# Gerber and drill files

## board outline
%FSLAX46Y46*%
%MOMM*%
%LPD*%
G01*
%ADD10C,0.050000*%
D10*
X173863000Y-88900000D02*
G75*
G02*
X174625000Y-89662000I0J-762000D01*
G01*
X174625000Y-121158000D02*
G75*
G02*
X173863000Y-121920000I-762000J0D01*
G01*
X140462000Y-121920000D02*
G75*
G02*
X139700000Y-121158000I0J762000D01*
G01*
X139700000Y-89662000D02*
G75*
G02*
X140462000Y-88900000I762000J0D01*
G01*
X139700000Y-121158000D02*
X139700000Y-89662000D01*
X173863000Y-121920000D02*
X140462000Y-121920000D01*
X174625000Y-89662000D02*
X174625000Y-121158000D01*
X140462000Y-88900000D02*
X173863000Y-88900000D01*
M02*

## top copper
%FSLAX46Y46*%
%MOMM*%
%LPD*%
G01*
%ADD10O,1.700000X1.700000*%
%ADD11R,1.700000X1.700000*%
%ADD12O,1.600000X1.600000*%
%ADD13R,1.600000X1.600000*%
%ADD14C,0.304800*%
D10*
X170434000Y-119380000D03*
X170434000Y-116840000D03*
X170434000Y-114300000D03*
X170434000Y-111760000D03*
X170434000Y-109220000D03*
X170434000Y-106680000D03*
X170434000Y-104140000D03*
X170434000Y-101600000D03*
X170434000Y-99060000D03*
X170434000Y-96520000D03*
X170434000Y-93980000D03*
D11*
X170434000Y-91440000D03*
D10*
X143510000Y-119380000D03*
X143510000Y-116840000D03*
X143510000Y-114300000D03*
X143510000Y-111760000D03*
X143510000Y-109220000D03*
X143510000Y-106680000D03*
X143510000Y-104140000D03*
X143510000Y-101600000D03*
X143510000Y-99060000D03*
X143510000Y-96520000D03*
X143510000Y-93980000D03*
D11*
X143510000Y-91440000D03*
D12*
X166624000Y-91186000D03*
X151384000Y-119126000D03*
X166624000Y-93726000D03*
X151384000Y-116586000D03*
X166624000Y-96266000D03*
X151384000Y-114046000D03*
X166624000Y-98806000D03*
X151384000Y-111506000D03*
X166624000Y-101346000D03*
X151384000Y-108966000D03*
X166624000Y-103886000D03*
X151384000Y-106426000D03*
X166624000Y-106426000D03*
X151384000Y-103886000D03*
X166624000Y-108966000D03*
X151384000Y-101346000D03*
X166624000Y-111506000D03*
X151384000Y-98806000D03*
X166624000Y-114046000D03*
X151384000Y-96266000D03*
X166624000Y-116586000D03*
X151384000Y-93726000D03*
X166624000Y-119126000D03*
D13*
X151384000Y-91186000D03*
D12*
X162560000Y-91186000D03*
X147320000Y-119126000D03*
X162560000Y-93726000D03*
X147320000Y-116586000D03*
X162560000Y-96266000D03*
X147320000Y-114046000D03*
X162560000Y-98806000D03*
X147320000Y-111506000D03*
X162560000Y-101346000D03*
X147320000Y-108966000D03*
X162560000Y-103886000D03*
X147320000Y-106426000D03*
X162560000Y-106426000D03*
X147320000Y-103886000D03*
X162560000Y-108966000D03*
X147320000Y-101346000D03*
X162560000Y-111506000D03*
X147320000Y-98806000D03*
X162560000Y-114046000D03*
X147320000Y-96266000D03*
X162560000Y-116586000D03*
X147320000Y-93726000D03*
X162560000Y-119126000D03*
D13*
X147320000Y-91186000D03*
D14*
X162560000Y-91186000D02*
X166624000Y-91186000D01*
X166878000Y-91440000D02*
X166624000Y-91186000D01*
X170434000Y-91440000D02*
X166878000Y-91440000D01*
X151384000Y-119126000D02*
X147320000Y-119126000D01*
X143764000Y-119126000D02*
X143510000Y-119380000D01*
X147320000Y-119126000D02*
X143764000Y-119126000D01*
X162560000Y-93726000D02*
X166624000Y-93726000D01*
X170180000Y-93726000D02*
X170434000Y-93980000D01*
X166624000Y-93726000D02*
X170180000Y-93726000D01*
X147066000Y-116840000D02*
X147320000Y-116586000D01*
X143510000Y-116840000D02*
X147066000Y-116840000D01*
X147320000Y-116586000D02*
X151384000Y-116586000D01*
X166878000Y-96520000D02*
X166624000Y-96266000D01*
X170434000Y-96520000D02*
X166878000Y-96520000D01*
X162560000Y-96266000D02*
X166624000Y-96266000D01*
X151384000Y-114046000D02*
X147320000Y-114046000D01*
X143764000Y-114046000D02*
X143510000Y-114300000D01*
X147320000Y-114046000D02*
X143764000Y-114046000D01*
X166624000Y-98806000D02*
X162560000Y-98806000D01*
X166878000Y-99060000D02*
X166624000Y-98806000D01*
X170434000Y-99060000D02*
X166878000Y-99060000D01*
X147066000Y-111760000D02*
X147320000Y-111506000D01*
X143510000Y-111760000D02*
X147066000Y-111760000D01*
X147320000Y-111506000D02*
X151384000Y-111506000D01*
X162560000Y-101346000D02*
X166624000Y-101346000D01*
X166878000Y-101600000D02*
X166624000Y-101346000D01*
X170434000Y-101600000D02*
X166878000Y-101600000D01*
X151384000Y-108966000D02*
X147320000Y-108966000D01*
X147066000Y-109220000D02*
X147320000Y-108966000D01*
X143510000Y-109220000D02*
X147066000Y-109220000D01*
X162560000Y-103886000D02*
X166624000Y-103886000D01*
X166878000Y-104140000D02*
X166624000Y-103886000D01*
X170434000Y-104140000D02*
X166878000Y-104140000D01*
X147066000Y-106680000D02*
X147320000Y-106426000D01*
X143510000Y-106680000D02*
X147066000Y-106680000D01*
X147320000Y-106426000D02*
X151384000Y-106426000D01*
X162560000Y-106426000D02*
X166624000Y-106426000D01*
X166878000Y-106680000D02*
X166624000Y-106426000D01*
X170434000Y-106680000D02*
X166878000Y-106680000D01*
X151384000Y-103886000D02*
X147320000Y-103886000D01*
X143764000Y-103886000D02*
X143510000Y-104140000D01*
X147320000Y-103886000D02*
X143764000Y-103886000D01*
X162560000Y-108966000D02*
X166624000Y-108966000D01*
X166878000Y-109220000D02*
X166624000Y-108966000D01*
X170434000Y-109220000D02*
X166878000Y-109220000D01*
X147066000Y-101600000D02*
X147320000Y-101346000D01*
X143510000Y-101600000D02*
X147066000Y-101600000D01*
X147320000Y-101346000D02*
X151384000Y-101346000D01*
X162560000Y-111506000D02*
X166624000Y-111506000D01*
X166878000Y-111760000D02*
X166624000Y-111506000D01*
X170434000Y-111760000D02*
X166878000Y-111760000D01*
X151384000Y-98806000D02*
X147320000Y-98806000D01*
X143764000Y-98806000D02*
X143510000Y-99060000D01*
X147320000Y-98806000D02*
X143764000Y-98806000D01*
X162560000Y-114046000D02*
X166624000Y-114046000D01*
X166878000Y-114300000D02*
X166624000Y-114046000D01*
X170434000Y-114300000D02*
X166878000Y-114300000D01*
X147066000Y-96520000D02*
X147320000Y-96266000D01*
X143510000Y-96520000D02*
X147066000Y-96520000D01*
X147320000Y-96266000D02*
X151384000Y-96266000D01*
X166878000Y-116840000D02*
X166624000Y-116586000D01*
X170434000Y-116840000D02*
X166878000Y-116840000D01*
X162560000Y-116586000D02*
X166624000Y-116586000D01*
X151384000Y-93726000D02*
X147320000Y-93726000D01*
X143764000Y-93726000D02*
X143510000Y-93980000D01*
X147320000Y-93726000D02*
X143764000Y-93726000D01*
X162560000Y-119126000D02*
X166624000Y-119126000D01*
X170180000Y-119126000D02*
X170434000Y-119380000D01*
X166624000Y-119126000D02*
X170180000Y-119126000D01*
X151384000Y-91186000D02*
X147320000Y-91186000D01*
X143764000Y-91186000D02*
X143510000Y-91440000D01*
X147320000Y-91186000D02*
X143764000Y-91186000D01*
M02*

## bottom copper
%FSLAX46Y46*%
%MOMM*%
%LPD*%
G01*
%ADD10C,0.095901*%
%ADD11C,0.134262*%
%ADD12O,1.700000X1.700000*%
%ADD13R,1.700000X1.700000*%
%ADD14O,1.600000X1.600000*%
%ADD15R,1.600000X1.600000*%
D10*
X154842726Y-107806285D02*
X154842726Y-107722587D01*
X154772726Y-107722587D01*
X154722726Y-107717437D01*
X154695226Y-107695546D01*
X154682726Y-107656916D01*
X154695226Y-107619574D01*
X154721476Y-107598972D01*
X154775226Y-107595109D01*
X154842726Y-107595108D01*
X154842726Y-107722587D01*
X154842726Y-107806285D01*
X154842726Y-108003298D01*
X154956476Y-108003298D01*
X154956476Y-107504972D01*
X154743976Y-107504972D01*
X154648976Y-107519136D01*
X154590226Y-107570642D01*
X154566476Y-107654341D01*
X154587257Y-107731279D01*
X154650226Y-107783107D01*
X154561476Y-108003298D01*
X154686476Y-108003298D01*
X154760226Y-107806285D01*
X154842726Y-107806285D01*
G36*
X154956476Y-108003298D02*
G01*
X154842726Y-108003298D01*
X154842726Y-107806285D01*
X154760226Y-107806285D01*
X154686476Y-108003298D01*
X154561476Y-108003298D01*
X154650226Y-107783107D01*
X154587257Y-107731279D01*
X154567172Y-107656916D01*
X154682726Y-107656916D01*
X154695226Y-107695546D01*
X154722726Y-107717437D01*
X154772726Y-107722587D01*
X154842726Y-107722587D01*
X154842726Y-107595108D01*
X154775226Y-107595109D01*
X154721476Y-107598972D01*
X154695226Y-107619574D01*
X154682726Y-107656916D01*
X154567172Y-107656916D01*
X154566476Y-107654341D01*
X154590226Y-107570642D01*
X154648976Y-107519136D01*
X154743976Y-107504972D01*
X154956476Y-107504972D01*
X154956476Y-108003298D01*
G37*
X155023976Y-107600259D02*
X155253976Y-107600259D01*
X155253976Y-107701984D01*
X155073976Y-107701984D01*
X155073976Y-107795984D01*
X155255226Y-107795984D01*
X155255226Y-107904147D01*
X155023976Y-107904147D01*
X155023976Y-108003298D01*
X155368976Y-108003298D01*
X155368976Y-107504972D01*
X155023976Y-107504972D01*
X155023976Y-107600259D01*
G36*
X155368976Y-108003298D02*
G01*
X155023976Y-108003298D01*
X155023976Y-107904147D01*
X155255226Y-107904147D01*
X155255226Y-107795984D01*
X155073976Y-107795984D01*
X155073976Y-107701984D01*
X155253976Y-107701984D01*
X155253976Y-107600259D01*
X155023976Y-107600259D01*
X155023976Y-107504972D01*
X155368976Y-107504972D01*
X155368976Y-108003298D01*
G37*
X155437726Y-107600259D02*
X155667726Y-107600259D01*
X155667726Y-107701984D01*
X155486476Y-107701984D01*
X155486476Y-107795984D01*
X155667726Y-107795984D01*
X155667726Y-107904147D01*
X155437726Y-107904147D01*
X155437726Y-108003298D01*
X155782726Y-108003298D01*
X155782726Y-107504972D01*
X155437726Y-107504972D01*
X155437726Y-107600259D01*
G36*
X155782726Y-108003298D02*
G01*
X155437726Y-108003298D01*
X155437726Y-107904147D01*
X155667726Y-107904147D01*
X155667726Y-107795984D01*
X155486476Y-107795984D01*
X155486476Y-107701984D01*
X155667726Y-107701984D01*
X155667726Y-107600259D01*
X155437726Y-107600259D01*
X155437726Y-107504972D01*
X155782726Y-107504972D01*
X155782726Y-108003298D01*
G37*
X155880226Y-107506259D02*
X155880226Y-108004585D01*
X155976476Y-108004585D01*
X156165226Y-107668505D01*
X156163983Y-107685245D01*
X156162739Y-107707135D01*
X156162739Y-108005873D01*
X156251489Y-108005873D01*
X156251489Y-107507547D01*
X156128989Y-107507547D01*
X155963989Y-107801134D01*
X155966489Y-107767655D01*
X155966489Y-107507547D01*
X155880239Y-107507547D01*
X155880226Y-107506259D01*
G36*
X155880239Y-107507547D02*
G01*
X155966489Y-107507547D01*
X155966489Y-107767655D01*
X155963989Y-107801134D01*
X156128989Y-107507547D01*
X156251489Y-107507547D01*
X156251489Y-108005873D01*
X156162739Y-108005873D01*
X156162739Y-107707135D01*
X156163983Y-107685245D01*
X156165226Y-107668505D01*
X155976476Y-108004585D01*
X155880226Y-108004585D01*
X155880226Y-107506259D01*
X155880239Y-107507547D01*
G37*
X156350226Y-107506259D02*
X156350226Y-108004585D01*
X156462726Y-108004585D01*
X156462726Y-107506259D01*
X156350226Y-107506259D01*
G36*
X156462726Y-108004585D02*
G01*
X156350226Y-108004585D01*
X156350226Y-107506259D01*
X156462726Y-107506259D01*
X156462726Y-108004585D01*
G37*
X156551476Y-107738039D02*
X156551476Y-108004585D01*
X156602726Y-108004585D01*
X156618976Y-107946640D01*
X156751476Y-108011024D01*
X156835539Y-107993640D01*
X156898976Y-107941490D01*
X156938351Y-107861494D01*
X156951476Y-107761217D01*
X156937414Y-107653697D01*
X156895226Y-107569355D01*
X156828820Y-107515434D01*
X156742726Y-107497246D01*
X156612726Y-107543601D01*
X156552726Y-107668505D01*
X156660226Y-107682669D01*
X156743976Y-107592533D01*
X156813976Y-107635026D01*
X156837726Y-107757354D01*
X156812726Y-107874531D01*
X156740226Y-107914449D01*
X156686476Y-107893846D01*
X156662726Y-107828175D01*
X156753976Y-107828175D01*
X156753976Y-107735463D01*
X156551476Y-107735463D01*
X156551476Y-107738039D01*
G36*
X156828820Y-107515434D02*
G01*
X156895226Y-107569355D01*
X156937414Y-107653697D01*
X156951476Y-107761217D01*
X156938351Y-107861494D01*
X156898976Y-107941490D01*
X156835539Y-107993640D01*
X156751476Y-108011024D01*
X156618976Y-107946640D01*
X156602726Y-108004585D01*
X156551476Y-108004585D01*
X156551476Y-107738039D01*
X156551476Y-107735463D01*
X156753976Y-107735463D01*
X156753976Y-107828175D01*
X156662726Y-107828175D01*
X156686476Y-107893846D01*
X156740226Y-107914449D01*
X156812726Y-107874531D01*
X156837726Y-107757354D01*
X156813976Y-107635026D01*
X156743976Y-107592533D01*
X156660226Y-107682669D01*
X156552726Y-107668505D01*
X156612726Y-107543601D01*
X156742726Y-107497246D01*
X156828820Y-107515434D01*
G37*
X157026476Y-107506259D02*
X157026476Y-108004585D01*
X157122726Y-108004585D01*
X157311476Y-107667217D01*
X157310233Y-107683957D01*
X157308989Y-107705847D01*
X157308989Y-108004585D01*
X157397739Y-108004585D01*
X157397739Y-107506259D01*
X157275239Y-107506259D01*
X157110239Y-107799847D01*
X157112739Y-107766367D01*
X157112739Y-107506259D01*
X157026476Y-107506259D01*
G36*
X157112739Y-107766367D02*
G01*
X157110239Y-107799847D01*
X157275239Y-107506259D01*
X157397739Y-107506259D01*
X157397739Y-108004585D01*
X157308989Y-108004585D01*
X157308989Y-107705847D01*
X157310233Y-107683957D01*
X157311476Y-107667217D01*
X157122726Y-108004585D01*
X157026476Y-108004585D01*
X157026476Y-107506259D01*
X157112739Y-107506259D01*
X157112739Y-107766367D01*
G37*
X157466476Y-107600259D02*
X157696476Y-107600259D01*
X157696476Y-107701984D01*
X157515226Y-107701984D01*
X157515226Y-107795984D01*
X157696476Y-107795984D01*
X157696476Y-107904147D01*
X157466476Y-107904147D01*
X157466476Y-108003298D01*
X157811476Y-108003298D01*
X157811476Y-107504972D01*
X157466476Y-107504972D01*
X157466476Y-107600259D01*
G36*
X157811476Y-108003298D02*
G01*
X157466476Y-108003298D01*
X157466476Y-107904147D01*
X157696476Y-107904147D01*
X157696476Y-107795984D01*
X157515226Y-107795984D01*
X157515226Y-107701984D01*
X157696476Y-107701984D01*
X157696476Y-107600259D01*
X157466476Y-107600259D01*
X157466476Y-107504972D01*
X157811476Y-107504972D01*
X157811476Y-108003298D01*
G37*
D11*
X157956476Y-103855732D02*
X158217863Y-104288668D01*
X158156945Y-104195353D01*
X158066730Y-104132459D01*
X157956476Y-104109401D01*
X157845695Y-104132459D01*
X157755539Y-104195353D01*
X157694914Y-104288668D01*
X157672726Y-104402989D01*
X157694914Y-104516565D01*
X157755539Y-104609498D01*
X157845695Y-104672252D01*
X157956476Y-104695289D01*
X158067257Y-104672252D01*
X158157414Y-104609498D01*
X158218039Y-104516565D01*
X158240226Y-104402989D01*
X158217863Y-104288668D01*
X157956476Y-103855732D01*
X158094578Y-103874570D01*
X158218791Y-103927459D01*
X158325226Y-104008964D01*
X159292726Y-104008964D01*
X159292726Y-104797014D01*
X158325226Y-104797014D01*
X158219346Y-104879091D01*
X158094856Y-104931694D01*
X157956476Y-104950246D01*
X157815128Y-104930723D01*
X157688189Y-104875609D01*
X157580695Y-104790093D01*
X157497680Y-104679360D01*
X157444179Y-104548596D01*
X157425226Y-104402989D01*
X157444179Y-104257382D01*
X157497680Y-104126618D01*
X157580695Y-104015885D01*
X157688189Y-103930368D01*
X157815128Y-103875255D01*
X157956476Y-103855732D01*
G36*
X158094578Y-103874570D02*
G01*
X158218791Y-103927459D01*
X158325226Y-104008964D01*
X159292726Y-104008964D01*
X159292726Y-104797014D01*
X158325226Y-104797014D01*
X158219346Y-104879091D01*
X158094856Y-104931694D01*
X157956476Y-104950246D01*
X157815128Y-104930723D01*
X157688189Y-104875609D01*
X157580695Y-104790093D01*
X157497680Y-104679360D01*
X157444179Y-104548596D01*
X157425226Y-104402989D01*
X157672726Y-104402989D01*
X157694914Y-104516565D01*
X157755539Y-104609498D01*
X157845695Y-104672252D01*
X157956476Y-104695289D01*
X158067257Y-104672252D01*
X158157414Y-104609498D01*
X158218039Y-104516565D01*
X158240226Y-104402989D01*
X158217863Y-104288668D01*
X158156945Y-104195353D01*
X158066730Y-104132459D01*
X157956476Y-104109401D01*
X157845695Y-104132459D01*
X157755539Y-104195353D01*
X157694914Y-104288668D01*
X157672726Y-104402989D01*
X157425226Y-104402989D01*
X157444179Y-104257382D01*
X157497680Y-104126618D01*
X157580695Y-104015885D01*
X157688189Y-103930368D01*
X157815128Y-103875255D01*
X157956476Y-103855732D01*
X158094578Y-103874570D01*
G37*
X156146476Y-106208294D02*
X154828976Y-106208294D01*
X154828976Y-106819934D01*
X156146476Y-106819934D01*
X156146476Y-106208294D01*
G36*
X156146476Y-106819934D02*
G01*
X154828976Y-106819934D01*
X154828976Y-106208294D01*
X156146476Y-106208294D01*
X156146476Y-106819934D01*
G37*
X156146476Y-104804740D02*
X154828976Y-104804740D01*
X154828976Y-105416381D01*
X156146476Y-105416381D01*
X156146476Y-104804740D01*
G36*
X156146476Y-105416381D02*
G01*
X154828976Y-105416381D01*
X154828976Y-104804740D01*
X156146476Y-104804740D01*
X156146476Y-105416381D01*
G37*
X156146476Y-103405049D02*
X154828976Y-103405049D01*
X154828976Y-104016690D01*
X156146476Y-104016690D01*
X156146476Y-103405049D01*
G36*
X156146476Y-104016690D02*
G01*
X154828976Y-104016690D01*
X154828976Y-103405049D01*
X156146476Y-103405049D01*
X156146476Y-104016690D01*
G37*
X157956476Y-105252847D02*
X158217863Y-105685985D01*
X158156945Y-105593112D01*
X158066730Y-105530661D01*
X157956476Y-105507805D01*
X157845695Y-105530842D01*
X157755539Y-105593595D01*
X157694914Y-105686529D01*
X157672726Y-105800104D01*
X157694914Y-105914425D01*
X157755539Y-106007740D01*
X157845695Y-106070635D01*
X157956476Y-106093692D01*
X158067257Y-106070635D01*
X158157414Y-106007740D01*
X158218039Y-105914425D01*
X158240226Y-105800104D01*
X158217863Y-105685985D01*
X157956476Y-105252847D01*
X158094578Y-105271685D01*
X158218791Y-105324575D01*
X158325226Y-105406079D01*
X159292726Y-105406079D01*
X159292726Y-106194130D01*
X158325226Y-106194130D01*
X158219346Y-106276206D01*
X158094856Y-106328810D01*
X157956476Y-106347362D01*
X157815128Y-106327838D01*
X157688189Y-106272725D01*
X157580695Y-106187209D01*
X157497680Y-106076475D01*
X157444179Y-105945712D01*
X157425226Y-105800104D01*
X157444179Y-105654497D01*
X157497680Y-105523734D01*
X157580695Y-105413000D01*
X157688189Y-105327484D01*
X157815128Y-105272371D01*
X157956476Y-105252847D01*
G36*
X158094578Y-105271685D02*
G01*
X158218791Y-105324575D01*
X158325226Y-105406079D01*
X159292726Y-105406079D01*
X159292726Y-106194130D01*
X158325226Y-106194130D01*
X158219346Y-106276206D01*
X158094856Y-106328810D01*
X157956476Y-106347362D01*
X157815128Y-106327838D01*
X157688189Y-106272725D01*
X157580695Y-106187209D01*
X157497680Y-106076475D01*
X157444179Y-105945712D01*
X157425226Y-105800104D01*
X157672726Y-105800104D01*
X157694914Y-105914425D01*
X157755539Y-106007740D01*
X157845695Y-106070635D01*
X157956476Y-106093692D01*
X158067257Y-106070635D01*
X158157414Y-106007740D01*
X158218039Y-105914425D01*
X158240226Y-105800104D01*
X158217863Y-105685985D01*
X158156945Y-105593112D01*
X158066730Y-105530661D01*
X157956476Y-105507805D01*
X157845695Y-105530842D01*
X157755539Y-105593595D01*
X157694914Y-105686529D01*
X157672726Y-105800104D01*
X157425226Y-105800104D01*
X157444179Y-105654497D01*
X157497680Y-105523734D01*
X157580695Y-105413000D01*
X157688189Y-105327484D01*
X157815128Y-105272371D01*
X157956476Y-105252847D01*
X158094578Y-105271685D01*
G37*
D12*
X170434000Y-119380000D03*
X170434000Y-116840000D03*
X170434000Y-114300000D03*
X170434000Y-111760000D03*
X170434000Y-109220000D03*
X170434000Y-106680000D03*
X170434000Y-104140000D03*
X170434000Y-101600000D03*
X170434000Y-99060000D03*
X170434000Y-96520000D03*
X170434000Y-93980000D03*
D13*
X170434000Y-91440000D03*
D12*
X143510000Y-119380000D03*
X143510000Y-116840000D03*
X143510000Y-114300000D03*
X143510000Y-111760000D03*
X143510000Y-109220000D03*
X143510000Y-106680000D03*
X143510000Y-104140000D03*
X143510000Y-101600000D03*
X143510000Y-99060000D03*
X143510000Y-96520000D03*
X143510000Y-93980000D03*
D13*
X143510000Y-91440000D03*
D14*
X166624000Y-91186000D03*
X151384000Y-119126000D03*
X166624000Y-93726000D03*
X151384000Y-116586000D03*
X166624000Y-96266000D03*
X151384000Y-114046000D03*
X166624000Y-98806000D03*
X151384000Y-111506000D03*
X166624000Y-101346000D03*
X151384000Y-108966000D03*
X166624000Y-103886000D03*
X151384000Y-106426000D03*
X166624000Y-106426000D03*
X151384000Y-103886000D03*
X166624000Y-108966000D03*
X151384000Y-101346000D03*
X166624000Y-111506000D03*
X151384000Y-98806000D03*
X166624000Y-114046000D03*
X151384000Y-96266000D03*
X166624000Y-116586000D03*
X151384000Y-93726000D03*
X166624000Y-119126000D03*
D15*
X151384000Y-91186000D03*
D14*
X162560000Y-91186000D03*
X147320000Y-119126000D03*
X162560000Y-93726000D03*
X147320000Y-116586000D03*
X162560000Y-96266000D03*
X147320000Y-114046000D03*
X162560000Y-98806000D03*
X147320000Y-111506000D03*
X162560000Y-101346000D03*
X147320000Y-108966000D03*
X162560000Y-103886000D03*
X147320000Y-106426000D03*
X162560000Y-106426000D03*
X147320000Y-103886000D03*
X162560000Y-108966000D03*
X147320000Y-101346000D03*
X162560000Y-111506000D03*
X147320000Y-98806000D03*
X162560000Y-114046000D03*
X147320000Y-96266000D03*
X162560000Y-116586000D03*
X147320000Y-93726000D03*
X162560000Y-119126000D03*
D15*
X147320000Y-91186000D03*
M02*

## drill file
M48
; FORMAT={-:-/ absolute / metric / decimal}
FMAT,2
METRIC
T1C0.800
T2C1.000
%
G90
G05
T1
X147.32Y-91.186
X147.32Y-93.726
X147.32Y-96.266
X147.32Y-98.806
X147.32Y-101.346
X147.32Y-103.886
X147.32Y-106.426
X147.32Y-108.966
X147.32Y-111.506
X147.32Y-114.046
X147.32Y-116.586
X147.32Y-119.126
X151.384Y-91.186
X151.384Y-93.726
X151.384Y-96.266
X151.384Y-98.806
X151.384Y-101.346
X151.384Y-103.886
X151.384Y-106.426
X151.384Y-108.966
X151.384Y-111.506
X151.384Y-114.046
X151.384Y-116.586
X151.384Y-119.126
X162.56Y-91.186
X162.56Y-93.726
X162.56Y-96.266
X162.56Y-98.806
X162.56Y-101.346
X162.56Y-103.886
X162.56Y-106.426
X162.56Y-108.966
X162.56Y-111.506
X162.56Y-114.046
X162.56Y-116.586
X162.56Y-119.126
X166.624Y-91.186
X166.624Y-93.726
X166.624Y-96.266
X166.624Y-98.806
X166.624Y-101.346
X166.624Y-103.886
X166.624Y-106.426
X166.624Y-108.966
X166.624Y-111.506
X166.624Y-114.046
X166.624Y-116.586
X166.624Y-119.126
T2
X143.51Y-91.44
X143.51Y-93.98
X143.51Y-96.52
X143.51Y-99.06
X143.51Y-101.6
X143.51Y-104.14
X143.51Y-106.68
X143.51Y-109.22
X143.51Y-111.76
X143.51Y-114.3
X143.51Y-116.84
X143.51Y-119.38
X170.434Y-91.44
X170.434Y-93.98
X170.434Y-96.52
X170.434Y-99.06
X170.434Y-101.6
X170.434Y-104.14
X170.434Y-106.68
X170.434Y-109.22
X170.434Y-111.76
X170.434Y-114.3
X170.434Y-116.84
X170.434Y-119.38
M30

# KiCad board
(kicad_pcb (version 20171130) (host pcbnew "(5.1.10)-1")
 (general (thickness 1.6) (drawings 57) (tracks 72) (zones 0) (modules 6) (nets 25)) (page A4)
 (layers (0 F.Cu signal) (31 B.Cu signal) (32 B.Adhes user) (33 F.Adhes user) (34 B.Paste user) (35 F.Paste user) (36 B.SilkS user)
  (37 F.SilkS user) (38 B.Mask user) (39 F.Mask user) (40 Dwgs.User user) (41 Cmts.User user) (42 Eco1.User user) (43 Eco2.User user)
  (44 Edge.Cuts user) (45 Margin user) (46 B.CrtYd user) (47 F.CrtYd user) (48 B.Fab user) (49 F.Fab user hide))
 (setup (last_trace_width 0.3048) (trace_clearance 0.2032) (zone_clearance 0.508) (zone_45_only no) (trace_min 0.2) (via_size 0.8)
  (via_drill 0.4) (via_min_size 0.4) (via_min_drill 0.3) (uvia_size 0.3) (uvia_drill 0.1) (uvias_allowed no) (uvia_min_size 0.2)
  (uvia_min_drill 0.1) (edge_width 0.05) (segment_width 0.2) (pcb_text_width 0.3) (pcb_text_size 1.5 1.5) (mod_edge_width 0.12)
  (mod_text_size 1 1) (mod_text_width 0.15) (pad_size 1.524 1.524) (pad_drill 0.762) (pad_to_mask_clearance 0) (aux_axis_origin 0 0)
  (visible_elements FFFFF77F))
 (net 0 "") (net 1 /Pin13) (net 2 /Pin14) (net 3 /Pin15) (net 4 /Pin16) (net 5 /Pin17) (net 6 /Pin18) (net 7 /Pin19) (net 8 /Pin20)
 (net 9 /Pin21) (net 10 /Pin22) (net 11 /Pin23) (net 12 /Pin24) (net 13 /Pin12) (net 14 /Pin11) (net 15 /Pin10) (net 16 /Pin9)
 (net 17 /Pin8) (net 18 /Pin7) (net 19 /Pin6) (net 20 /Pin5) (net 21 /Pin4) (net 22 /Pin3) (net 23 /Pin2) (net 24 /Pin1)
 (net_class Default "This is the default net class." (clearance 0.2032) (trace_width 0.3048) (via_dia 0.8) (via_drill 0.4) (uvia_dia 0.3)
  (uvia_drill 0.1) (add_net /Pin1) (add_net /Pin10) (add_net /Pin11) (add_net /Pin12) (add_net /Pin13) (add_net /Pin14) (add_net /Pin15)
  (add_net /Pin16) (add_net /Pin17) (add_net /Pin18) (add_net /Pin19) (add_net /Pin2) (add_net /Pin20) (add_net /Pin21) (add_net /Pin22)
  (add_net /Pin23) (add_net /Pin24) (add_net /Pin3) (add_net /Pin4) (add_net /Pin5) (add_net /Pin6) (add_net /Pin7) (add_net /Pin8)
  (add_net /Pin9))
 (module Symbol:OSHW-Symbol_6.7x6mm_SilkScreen (layer B.Cu) (at 157.0736 95.6818 180)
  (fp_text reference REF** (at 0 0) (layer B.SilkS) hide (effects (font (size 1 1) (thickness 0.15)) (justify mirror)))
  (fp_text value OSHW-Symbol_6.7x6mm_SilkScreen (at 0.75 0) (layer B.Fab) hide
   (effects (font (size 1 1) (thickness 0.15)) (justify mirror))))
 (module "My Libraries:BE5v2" (layer B.Cu) (at 159.561476 103.011024 180)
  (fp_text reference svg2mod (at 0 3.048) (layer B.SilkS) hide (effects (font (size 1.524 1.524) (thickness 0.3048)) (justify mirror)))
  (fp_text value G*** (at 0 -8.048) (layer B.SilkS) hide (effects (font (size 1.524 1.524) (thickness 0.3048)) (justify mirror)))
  (fp_poly
   (pts (xy 4.71875 -4.795261) (xy 4.71875 -4.711563) (xy 4.78875 -4.711563) (xy 4.83875 -4.706413) (xy 4.86625 -4.684522)
    (xy 4.87875 -4.645892) (xy 4.86625 -4.60855) (xy 4.84 -4.587948) (xy 4.78625 -4.584085) (xy 4.71875 -4.584084) (xy 4.71875 -4.711563)
    (xy 4.71875 -4.795261) (xy 4.71875 -4.992274) (xy 4.605 -4.992274) (xy 4.605 -4.493948) (xy 4.8175 -4.493948) (xy 4.9125 -4.508112)
    (xy 4.97125 -4.559618) (xy 4.995 -4.643317) (xy 4.974219 -4.720255) (xy 4.91125 -4.772083) (xy 5 -4.992274) (xy 4.875 -4.992274)
    (xy 4.80125 -4.795261) (xy 4.71875 -4.795261))
   (layer B.Cu) (width 0.095901))
  (fp_poly
   (pts (xy 4.5375 -4.589235) (xy 4.3075 -4.589235) (xy 4.3075 -4.69096) (xy 4.4875 -4.69096) (xy 4.4875 -4.78496) (xy 4.30625 -4.78496)
    (xy 4.30625 -4.893123) (xy 4.5375 -4.893123) (xy 4.5375 -4.992274) (xy 4.1925 -4.992274) (xy 4.1925 -4.493948) (xy 4.5375 -4.493948)
    (xy 4.5375 -4.589235))
   (layer B.Cu) (width 0.095901))
  (fp_poly
   (pts (xy 4.12375 -4.589235) (xy 3.89375 -4.589235) (xy 3.89375 -4.69096) (xy 4.075 -4.69096) (xy 4.075 -4.78496) (xy 3.89375 -4.78496)
    (xy 3.89375 -4.893123) (xy 4.12375 -4.893123) (xy 4.12375 -4.992274) (xy 3.77875 -4.992274) (xy 3.77875 -4.493948)
    (xy 4.12375 -4.493948) (xy 4.12375 -4.589235))
   (layer B.Cu) (width 0.095901))
  (fp_poly
   (pts (xy 3.68125 -4.495235) (xy 3.68125 -4.993561) (xy 3.585 -4.993561) (xy 3.39625 -4.657481) (xy 3.397493 -4.674221)
    (xy 3.398737 -4.696111) (xy 3.398737 -4.994849) (xy 3.309987 -4.994849) (xy 3.309987 -4.496523) (xy 3.432487 -4.496523)
    (xy 3.597487 -4.79011) (xy 3.594987 -4.756631) (xy 3.594987 -4.496523) (xy 3.681237 -4.496523) (xy 3.68125 -4.495235))
   (layer B.Cu) (width 0.095901))
  (fp_poly
   (pts (xy 3.21125 -4.495235) (xy 3.21125 -4.993561) (xy 3.09875 -4.993561) (xy 3.09875 -4.495235) (xy 3.21125 -4.495235)) (layer B.Cu)
   (width 0.095901))
  (fp_poly
   (pts (xy 3.01 -4.727015) (xy 3.01 -4.993561) (xy 2.95875 -4.993561) (xy 2.9425 -4.935616) (xy 2.81 -5) (xy 2.725937 -4.982616)
    (xy 2.6625 -4.930466) (xy 2.623125 -4.85047) (xy 2.61 -4.750193) (xy 2.624062 -4.642673) (xy 2.66625 -4.558331) (xy 2.732656 -4.50441)
    (xy 2.81875 -4.486222) (xy 2.94875 -4.532577) (xy 3.00875 -4.657481) (xy 2.90125 -4.671645) (xy 2.8175 -4.581509) (xy 2.7475 -4.624002)
    (xy 2.72375 -4.74633) (xy 2.74875 -4.863507) (xy 2.82125 -4.903425) (xy 2.875 -4.882822) (xy 2.89875 -4.817151) (xy 2.8075 -4.817151)
    (xy 2.8075 -4.724439) (xy 3.01 -4.724439) (xy 3.01 -4.727015))
   (layer B.Cu) (width 0.095901))
  (fp_poly
   (pts (xy 2.535 -4.495235) (xy 2.535 -4.993561) (xy 2.43875 -4.993561) (xy 2.25 -4.656193) (xy 2.251243 -4.672933) (xy 2.252487 -4.694823)
    (xy 2.252487 -4.993561) (xy 2.163737 -4.993561) (xy 2.163737 -4.495235) (xy 2.286237 -4.495235) (xy 2.451237 -4.788823)
    (xy 2.448737 -4.755343) (xy 2.448737 -4.495235) (xy 2.535 -4.495235))
   (layer B.Cu) (width 0.095901))
  (fp_poly
   (pts (xy 2.095 -4.589235) (xy 1.865 -4.589235) (xy 1.865 -4.69096) (xy 2.04625 -4.69096) (xy 2.04625 -4.78496) (xy 1.865 -4.78496)
    (xy 1.865 -4.893123) (xy 2.095 -4.893123) (xy 2.095 -4.992274) (xy 1.75 -4.992274) (xy 1.75 -4.493948) (xy 2.095 -4.493948)
    (xy 2.095 -4.589235))
   (layer B.Cu) (width 0.095901))
  (fp_poly
   (pts (xy 1.605 -0.844708) (xy 1.343613 -1.277644) (xy 1.404531 -1.184329) (xy 1.494746 -1.121435) (xy 1.605 -1.098377)
    (xy 1.715781 -1.121435) (xy 1.805937 -1.184329) (xy 1.866562 -1.277644) (xy 1.88875 -1.391965) (xy 1.866562 -1.505541)
    (xy 1.805937 -1.598474) (xy 1.715781 -1.661228) (xy 1.605 -1.684265) (xy 1.494219 -1.661228) (xy 1.404062 -1.598474)
    (xy 1.343437 -1.505541) (xy 1.32125 -1.391965) (xy 1.343613 -1.277644) (xy 1.605 -0.844708) (xy 1.466898 -0.863546)
    (xy 1.342685 -0.916435) (xy 1.23625 -0.99794) (xy 0.26875 -0.99794) (xy 0.26875 -1.78599) (xy 1.23625 -1.78599) (xy 1.34213 -1.868067)
    (xy 1.46662 -1.92067) (xy 1.605 -1.939222) (xy 1.746348 -1.919699) (xy 1.873287 -1.864585) (xy 1.980781 -1.779069)
    (xy 2.063796 -1.668336) (xy 2.117297 -1.537572) (xy 2.13625 -1.391965) (xy 2.117297 -1.246358) (xy 2.063796 -1.115594)
    (xy 1.980781 -1.004861) (xy 1.873287 -0.919344) (xy 1.746348 -0.864231) (xy 1.605 -0.844708))
   (layer B.Cu) (width 0.134262))
  (fp_poly
   (pts (xy 3.415 -3.19727) (xy 4.7325 -3.19727) (xy 4.7325 -3.80891) (xy 3.415 -3.80891) (xy 3.415 -3.19727)) (layer B.Cu) (width 0.134262))
  (fp_poly
   (pts (xy 3.415 -1.793716) (xy 4.7325 -1.793716) (xy 4.7325 -2.405357) (xy 3.415 -2.405357) (xy 3.415 -1.793716)) (layer B.Cu)
   (width 0.134262))
  (fp_poly
   (pts (xy 3.415 -0.394025) (xy 4.7325 -0.394025) (xy 4.7325 -1.005666) (xy 3.415 -1.005666) (xy 3.415 -0.394025)) (layer B.Cu)
   (width 0.134262))
  (fp_poly
   (pts (xy 1.605 -2.241823) (xy 1.343613 -2.674961) (xy 1.404531 -2.582088) (xy 1.494746 -2.519637) (xy 1.605 -2.496781)
    (xy 1.715781 -2.519818) (xy 1.805937 -2.582571) (xy 1.866562 -2.675505) (xy 1.88875 -2.78908) (xy 1.866562 -2.903401)
    (xy 1.805937 -2.996716) (xy 1.715781 -3.059611) (xy 1.605 -3.082668) (xy 1.494219 -3.059611) (xy 1.404062 -2.996716)
    (xy 1.343437 -2.903401) (xy 1.32125 -2.78908) (xy 1.343613 -2.674961) (xy 1.605 -2.241823) (xy 1.466898 -2.260661)
    (xy 1.342685 -2.313551) (xy 1.23625 -2.395055) (xy 0.26875 -2.395055) (xy 0.26875 -3.183106) (xy 1.23625 -3.183106)
    (xy 1.34213 -3.265182) (xy 1.46662 -3.317786) (xy 1.605 -3.336338) (xy 1.746348 -3.316814) (xy 1.873287 -3.261701)
    (xy 1.980781 -3.176185) (xy 2.063796 -3.065451) (xy 2.117297 -2.934688) (xy 2.13625 -2.78908) (xy 2.117297 -2.643473)
    (xy 2.063796 -2.51271) (xy 1.980781 -2.401976) (xy 1.873287 -2.31646) (xy 1.746348 -2.261347) (xy 1.605 -2.241823))
   (layer B.Cu) (width 0.134262)))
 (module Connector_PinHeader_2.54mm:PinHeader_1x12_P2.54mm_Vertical (layer F.Cu) (at 170.434 91.44)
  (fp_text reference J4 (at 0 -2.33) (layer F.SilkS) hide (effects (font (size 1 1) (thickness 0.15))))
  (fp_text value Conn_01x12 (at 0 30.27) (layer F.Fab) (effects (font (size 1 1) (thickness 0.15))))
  (pad 12 thru_hole oval (at 0 27.94) (size 1.7 1.7) (drill 1) (layers *.Cu *.Mask) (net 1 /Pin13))
  (pad 11 thru_hole oval (at 0 25.4) (size 1.7 1.7) (drill 1) (layers *.Cu *.Mask) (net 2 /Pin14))
  (pad 10 thru_hole oval (at 0 22.86) (size 1.7 1.7) (drill 1) (layers *.Cu *.Mask) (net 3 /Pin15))
  (pad 9 thru_hole oval (at 0 20.32) (size 1.7 1.7) (drill 1) (layers *.Cu *.Mask) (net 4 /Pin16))
  (pad 8 thru_hole oval (at 0 17.78) (size 1.7 1.7) (drill 1) (layers *.Cu *.Mask) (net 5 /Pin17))
  (pad 7 thru_hole oval (at 0 15.24) (size 1.7 1.7) (drill 1) (layers *.Cu *.Mask) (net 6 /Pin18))
  (pad 6 thru_hole oval (at 0 12.7) (size 1.7 1.7) (drill 1) (layers *.Cu *.Mask) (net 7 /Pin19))
  (pad 5 thru_hole oval (at 0 10.16) (size 1.7 1.7) (drill 1) (layers *.Cu *.Mask) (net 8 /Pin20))
  (pad 4 thru_hole oval (at 0 7.62) (size 1.7 1.7) (drill 1) (layers *.Cu *.Mask) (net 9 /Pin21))
  (pad 3 thru_hole oval (at 0 5.08) (size 1.7 1.7) (drill 1) (layers *.Cu *.Mask) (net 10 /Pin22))
  (pad 2 thru_hole oval (at 0 2.54) (size 1.7 1.7) (drill 1) (layers *.Cu *.Mask) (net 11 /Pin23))
  (pad 1 thru_hole rect (at 0 0) (size 1.7 1.7) (drill 1) (layers *.Cu *.Mask) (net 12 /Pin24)))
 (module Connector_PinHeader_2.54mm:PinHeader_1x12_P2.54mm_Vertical (layer F.Cu) (at 143.51 91.44)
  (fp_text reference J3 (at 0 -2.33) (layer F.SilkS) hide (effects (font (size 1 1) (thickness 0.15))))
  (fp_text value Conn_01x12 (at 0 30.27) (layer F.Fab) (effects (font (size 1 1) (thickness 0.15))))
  (pad 12 thru_hole oval (at 0 27.94) (size 1.7 1.7) (drill 1) (layers *.Cu *.Mask) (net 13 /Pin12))
  (pad 11 thru_hole oval (at 0 25.4) (size 1.7 1.7) (drill 1) (layers *.Cu *.Mask) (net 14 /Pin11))
  (pad 10 thru_hole oval (at 0 22.86) (size 1.7 1.7) (drill 1) (layers *.Cu *.Mask) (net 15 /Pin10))
  (pad 9 thru_hole oval (at 0 20.32) (size 1.7 1.7) (drill 1) (layers *.Cu *.Mask) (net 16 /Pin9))
  (pad 8 thru_hole oval (at 0 17.78) (size 1.7 1.7) (drill 1) (layers *.Cu *.Mask) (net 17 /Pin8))
  (pad 7 thru_hole oval (at 0 15.24) (size 1.7 1.7) (drill 1) (layers *.Cu *.Mask) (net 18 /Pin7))
  (pad 6 thru_hole oval (at 0 12.7) (size 1.7 1.7) (drill 1) (layers *.Cu *.Mask) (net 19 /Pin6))
  (pad 5 thru_hole oval (at 0 10.16) (size 1.7 1.7) (drill 1) (layers *.Cu *.Mask) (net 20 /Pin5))
  (pad 4 thru_hole oval (at 0 7.62) (size 1.7 1.7) (drill 1) (layers *.Cu *.Mask) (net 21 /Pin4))
  (pad 3 thru_hole oval (at 0 5.08) (size 1.7 1.7) (drill 1) (layers *.Cu *.Mask) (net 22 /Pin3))
  (pad 2 thru_hole oval (at 0 2.54) (size 1.7 1.7) (drill 1) (layers *.Cu *.Mask) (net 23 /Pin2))
  (pad 1 thru_hole rect (at 0 0) (size 1.7 1.7) (drill 1) (layers *.Cu *.Mask) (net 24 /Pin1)))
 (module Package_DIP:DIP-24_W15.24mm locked (layer F.Cu) (at 151.384 91.186)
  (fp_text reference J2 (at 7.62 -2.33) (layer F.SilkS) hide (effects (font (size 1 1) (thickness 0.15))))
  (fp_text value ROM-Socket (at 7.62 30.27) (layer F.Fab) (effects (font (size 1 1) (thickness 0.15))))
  (pad 24 thru_hole oval (at 15.24 0) (size 1.6 1.6) (drill 0.8) (layers *.Cu *.Mask) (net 12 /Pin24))
  (pad 12 thru_hole oval (at 0 27.94) (size 1.6 1.6) (drill 0.8) (layers *.Cu *.Mask) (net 13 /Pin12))
  (pad 23 thru_hole oval (at 15.24 2.54) (size 1.6 1.6) (drill 0.8) (layers *.Cu *.Mask) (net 11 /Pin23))
  (pad 11 thru_hole oval (at 0 25.4) (size 1.6 1.6) (drill 0.8) (layers *.Cu *.Mask) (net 14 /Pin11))
  (pad 22 thru_hole oval (at 15.24 5.08) (size 1.6 1.6) (drill 0.8) (layers *.Cu *.Mask) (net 10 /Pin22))
  (pad 10 thru_hole oval (at 0 22.86) (size 1.6 1.6) (drill 0.8) (layers *.Cu *.Mask) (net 15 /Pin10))
  (pad 21 thru_hole oval (at 15.24 7.62) (size 1.6 1.6) (drill 0.8) (layers *.Cu *.Mask) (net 9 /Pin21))
  (pad 9 thru_hole oval (at 0 20.32) (size 1.6 1.6) (drill 0.8) (layers *.Cu *.Mask) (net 16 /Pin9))
  (pad 20 thru_hole oval (at 15.24 10.16) (size 1.6 1.6) (drill 0.8) (layers *.Cu *.Mask) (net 8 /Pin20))
  (pad 8 thru_hole oval (at 0 17.78) (size 1.6 1.6) (drill 0.8) (layers *.Cu *.Mask) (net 17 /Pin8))
  (pad 19 thru_hole oval (at 15.24 12.7) (size 1.6 1.6) (drill 0.8) (layers *.Cu *.Mask) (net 7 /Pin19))
  (pad 7 thru_hole oval (at 0 15.24) (size 1.6 1.6) (drill 0.8) (layers *.Cu *.Mask) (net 18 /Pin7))
  (pad 18 thru_hole oval (at 15.24 15.24) (size 1.6 1.6) (drill 0.8) (layers *.Cu *.Mask) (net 6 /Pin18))
  (pad 6 thru_hole oval (at 0 12.7) (size 1.6 1.6) (drill 0.8) (layers *.Cu *.Mask) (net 19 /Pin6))
  (pad 17 thru_hole oval (at 15.24 17.78) (size 1.6 1.6) (drill 0.8) (layers *.Cu *.Mask) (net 5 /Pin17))
  (pad 5 thru_hole oval (at 0 10.16) (size 1.6 1.6) (drill 0.8) (layers *.Cu *.Mask) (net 20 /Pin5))
  (pad 16 thru_hole oval (at 15.24 20.32) (size 1.6 1.6) (drill 0.8) (layers *.Cu *.Mask) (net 4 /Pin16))
  (pad 4 thru_hole oval (at 0 7.62) (size 1.6 1.6) (drill 0.8) (layers *.Cu *.Mask) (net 21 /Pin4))
  (pad 15 thru_hole oval (at 15.24 22.86) (size 1.6 1.6) (drill 0.8) (layers *.Cu *.Mask) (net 3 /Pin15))
  (pad 3 thru_hole oval (at 0 5.08) (size 1.6 1.6) (drill 0.8) (layers *.Cu *.Mask) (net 22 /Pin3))
  (pad 14 thru_hole oval (at 15.24 25.4) (size 1.6 1.6) (drill 0.8) (layers *.Cu *.Mask) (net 2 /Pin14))
  (pad 2 thru_hole oval (at 0 2.54) (size 1.6 1.6) (drill 0.8) (layers *.Cu *.Mask) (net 23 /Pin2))
  (pad 13 thru_hole oval (at 15.24 27.94) (size 1.6 1.6) (drill 0.8) (layers *.Cu *.Mask) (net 1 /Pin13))
  (pad 1 thru_hole rect (at 0 0) (size 1.6 1.6) (drill 0.8) (layers *.Cu *.Mask) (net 24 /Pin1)))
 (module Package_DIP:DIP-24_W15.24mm (layer F.Cu) (at 147.32 91.186)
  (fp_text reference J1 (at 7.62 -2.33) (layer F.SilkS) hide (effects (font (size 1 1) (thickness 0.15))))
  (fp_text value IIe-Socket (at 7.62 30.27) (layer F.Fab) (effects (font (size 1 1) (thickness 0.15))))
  (pad 24 thru_hole oval (at 15.24 0) (size 1.6 1.6) (drill 0.8) (layers *.Cu *.Mask) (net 12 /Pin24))
  (pad 12 thru_hole oval (at 0 27.94) (size 1.6 1.6) (drill 0.8) (layers *.Cu *.Mask) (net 13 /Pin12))
  (pad 23 thru_hole oval (at 15.24 2.54) (size 1.6 1.6) (drill 0.8) (layers *.Cu *.Mask) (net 11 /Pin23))
  (pad 11 thru_hole oval (at 0 25.4) (size 1.6 1.6) (drill 0.8) (layers *.Cu *.Mask) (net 14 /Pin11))
  (pad 22 thru_hole oval (at 15.24 5.08) (size 1.6 1.6) (drill 0.8) (layers *.Cu *.Mask) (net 10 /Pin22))
  (pad 10 thru_hole oval (at 0 22.86) (size 1.6 1.6) (drill 0.8) (layers *.Cu *.Mask) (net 15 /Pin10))
  (pad 21 thru_hole oval (at 15.24 7.62) (size 1.6 1.6) (drill 0.8) (layers *.Cu *.Mask) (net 9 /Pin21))
  (pad 9 thru_hole oval (at 0 20.32) (size 1.6 1.6) (drill 0.8) (layers *.Cu *.Mask) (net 16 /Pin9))
  (pad 20 thru_hole oval (at 15.24 10.16) (size 1.6 1.6) (drill 0.8) (layers *.Cu *.Mask) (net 8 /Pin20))
  (pad 8 thru_hole oval (at 0 17.78) (size 1.6 1.6) (drill 0.8) (layers *.Cu *.Mask) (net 17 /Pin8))
  (pad 19 thru_hole oval (at 15.24 12.7) (size 1.6 1.6) (drill 0.8) (layers *.Cu *.Mask) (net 7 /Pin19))
  (pad 7 thru_hole oval (at 0 15.24) (size 1.6 1.6) (drill 0.8) (layers *.Cu *.Mask) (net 18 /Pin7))
  (pad 18 thru_hole oval (at 15.24 15.24) (size 1.6 1.6) (drill 0.8) (layers *.Cu *.Mask) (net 6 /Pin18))
  (pad 6 thru_hole oval (at 0 12.7) (size 1.6 1.6) (drill 0.8) (layers *.Cu *.Mask) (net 19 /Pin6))
  (pad 17 thru_hole oval (at 15.24 17.78) (size 1.6 1.6) (drill 0.8) (layers *.Cu *.Mask) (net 5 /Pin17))
  (pad 5 thru_hole oval (at 0 10.16) (size 1.6 1.6) (drill 0.8) (layers *.Cu *.Mask) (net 20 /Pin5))
  (pad 16 thru_hole oval (at 15.24 20.32) (size 1.6 1.6) (drill 0.8) (layers *.Cu *.Mask) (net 4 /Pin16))
  (pad 4 thru_hole oval (at 0 7.62) (size 1.6 1.6) (drill 0.8) (layers *.Cu *.Mask) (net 21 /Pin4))
  (pad 15 thru_hole oval (at 15.24 22.86) (size 1.6 1.6) (drill 0.8) (layers *.Cu *.Mask) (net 3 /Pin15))
  (pad 3 thru_hole oval (at 0 5.08) (size 1.6 1.6) (drill 0.8) (layers *.Cu *.Mask) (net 22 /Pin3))
  (pad 14 thru_hole oval (at 15.24 25.4) (size 1.6 1.6) (drill 0.8) (layers *.Cu *.Mask) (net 2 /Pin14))
  (pad 2 thru_hole oval (at 0 2.54) (size 1.6 1.6) (drill 0.8) (layers *.Cu *.Mask) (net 23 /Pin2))
  (pad 13 thru_hole oval (at 15.24 27.94) (size 1.6 1.6) (drill 0.8) (layers *.Cu *.Mask) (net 1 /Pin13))
  (pad 1 thru_hole rect (at 0 0) (size 1.6 1.6) (drill 0.8) (layers *.Cu *.Mask) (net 24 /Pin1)))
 (gr_arc (start 173.863 89.662) (end 174.625 89.662) (angle -90) (layer Edge.Cuts) (width 0.05))
 (gr_arc (start 173.863 121.158) (end 173.863 121.92) (angle -90) (layer Edge.Cuts) (width 0.05))
 (gr_arc (start 140.462 121.158) (end 139.7 121.158) (angle -90) (layer Edge.Cuts) (width 0.05))
 (gr_arc (start 140.462 89.662) (end 140.462 88.9) (angle -90) (layer Edge.Cuts) (width 0.05))
 (gr_line (start 139.7 121.158) (end 139.7 89.662) (layer Edge.Cuts) (width 0.05))
 (gr_line (start 173.863 121.92) (end 140.462 121.92) (layer Edge.Cuts) (width 0.05))
 (gr_line (start 174.625 89.662) (end 174.625 121.158) (layer Edge.Cuts) (width 0.05))
 (gr_line (start 140.462 88.9) (end 173.863 88.9) (layer Edge.Cuts) (width 0.05))
 (segment (start 162.56 91.186) (end 166.624 91.186) (width 0.3048) (layer F.Cu) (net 12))
 (segment (start 166.878 91.44) (end 166.624 91.186) (width 0.3048) (layer F.Cu) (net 12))
 (segment (start 170.434 91.44) (end 166.878 91.44) (width 0.3048) (layer F.Cu) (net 12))
 (segment (start 151.384 119.126) (end 147.32 119.126) (width 0.3048) (layer F.Cu) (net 13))
 (segment (start 143.764 119.126) (end 143.51 119.38) (width 0.3048) (layer F.Cu) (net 13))
 (segment (start 147.32 119.126) (end 143.764 119.126) (width 0.3048) (layer F.Cu) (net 13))
 (segment (start 162.56 93.726) (end 166.624 93.726) (width 0.3048) (layer F.Cu) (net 11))
 (segment (start 170.18 93.726) (end 170.434 93.98) (width 0.3048) (layer F.Cu) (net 11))
 (segment (start 166.624 93.726) (end 170.18 93.726) (width 0.3048) (layer F.Cu) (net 11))
 (segment (start 147.066 116.84) (end 147.32 116.586) (width 0.3048) (layer F.Cu) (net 14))
 (segment (start 143.51 116.84) (end 147.066 116.84) (width 0.3048) (layer F.Cu) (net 14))
 (segment (start 147.32 116.586) (end 151.384 116.586) (width 0.3048) (layer F.Cu) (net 14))
 (segment (start 166.878 96.52) (end 166.624 96.266) (width 0.3048) (layer F.Cu) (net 10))
 (segment (start 170.434 96.52) (end 166.878 96.52) (width 0.3048) (layer F.Cu) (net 10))
 (segment (start 162.56 96.266) (end 166.624 96.266) (width 0.3048) (layer F.Cu) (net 10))
 (segment (start 151.384 114.046) (end 147.32 114.046) (width 0.3048) (layer F.Cu) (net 15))
 (segment (start 143.764 114.046) (end 143.51 114.3) (width 0.3048) (layer F.Cu) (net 15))
 (segment (start 147.32 114.046) (end 143.764 114.046) (width 0.3048) (layer F.Cu) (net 15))
 (segment (start 166.624 98.806) (end 162.56 98.806) (width 0.3048) (layer F.Cu) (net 9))
 (segment (start 166.878 99.06) (end 166.624 98.806) (width 0.3048) (layer F.Cu) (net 9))
 (segment (start 170.434 99.06) (end 166.878 99.06) (width 0.3048) (layer F.Cu) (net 9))
 (segment (start 147.066 111.76) (end 147.32 111.506) (width 0.3048) (layer F.Cu) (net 16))
 (segment (start 143.51 111.76) (end 147.066 111.76) (width 0.3048) (layer F.Cu) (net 16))
 (segment (start 147.32 111.506) (end 151.384 111.506) (width 0.3048) (layer F.Cu) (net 16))
 (segment (start 162.56 101.346) (end 166.624 101.346) (width 0.3048) (layer F.Cu) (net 8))
 (segment (start 166.878 101.6) (end 166.624 101.346) (width 0.3048) (layer F.Cu) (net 8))
 (segment (start 170.434 101.6) (end 166.878 101.6) (width 0.3048) (layer F.Cu) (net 8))
 (segment (start 151.384 108.966) (end 147.32 108.966) (width 0.3048) (layer F.Cu) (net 17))
 (segment (start 147.066 109.22) (end 147.32 108.966) (width 0.3048) (layer F.Cu) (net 17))
 (segment (start 143.51 109.22) (end 147.066 109.22) (width 0.3048) (layer F.Cu) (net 17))
 (segment (start 162.56 103.886) (end 166.624 103.886) (width 0.3048) (layer F.Cu) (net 7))
 (segment (start 166.878 104.14) (end 166.624 103.886) (width 0.3048) (layer F.Cu) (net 7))
 (segment (start 170.434 104.14) (end 166.878 104.14) (width 0.3048) (layer F.Cu) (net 7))
 (segment (start 147.066 106.68) (end 147.32 106.426) (width 0.3048) (layer F.Cu) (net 18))
 (segment (start 143.51 106.68) (end 147.066 106.68) (width 0.3048) (layer F.Cu) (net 18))
 (segment (start 147.32 106.426) (end 151.384 106.426) (width 0.3048) (layer F.Cu) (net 18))
 (segment (start 162.56 106.426) (end 166.624 106.426) (width 0.3048) (layer F.Cu) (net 6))
 (segment (start 166.878 106.68) (end 166.624 106.426) (width 0.3048) (layer F.Cu) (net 6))
 (segment (start 170.434 106.68) (end 166.878 106.68) (width 0.3048) (layer F.Cu) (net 6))
 (segment (start 151.384 103.886) (end 147.32 103.886) (width 0.3048) (layer F.Cu) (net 19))
 (segment (start 143.764 103.886) (end 143.51 104.14) (width 0.3048) (layer F.Cu) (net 19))
 (segment (start 147.32 103.886) (end 143.764 103.886) (width 0.3048) (layer F.Cu) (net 19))
 (segment (start 162.56 108.966) (end 166.624 108.966) (width 0.3048) (layer F.Cu) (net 5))
 (segment (start 166.878 109.22) (end 166.624 108.966) (width 0.3048) (layer F.Cu) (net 5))
 (segment (start 170.434 109.22) (end 166.878 109.22) (width 0.3048) (layer F.Cu) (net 5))
 (segment (start 147.066 101.6) (end 147.32 101.346) (width 0.3048) (layer F.Cu) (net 20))
 (segment (start 143.51 101.6) (end 147.066 101.6) (width 0.3048) (layer F.Cu) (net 20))
 (segment (start 147.32 101.346) (end 151.384 101.346) (width 0.3048) (layer F.Cu) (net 20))
 (segment (start 162.56 111.506) (end 166.624 111.506) (width 0.3048) (layer F.Cu) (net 4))
 (segment (start 166.878 111.76) (end 166.624 111.506) (width 0.3048) (layer F.Cu) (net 4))
 (segment (start 170.434 111.76) (end 166.878 111.76) (width 0.3048) (layer F.Cu) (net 4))
 (segment (start 151.384 98.806) (end 147.32 98.806) (width 0.3048) (layer F.Cu) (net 21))
 (segment (start 143.764 98.806) (end 143.51 99.06) (width 0.3048) (layer F.Cu) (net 21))
 (segment (start 147.32 98.806) (end 143.764 98.806) (width 0.3048) (layer F.Cu) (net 21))
 (segment (start 162.56 114.046) (end 166.624 114.046) (width 0.3048) (layer F.Cu) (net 3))
 (segment (start 166.878 114.3) (end 166.624 114.046) (width 0.3048) (layer F.Cu) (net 3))
 (segment (start 170.434 114.3) (end 166.878 114.3) (width 0.3048) (layer F.Cu) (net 3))
 (segment (start 147.066 96.52) (end 147.32 96.266) (width 0.3048) (layer F.Cu) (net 22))
 (segment (start 143.51 96.52) (end 147.066 96.52) (width 0.3048) (layer F.Cu) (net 22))
 (segment (start 147.32 96.266) (end 151.384 96.266) (width 0.3048) (layer F.Cu) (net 22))
 (segment (start 166.878 116.84) (end 166.624 116.586) (width 0.3048) (layer F.Cu) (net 2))
 (segment (start 170.434 116.84) (end 166.878 116.84) (width 0.3048) (layer F.Cu) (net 2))
 (segment (start 162.56 116.586) (end 166.624 116.586) (width 0.3048) (layer F.Cu) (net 2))
 (segment (start 151.384 93.726) (end 147.32 93.726) (width 0.3048) (layer F.Cu) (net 23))
 (segment (start 143.764 93.726) (end 143.51 93.98) (width 0.3048) (layer F.Cu) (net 23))
 (segment (start 147.32 93.726) (end 143.764 93.726) (width 0.3048) (layer F.Cu) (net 23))
 (segment (start 162.56 119.126) (end 166.624 119.126) (width 0.3048) (layer F.Cu) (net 1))
 (segment (start 170.18 119.126) (end 170.434 119.38) (width 0.3048) (layer F.Cu) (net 1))
 (segment (start 166.624 119.126) (end 170.18 119.126) (width 0.3048) (layer F.Cu) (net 1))
 (segment (start 151.384 91.186) (end 147.32 91.186) (width 0.3048) (layer F.Cu) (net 24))
 (segment (start 143.764 91.186) (end 143.51 91.44) (width 0.3048) (layer F.Cu) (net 24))
 (segment (start 147.32 91.186) (end 143.764 91.186) (width 0.3048) (layer F.Cu) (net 24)))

